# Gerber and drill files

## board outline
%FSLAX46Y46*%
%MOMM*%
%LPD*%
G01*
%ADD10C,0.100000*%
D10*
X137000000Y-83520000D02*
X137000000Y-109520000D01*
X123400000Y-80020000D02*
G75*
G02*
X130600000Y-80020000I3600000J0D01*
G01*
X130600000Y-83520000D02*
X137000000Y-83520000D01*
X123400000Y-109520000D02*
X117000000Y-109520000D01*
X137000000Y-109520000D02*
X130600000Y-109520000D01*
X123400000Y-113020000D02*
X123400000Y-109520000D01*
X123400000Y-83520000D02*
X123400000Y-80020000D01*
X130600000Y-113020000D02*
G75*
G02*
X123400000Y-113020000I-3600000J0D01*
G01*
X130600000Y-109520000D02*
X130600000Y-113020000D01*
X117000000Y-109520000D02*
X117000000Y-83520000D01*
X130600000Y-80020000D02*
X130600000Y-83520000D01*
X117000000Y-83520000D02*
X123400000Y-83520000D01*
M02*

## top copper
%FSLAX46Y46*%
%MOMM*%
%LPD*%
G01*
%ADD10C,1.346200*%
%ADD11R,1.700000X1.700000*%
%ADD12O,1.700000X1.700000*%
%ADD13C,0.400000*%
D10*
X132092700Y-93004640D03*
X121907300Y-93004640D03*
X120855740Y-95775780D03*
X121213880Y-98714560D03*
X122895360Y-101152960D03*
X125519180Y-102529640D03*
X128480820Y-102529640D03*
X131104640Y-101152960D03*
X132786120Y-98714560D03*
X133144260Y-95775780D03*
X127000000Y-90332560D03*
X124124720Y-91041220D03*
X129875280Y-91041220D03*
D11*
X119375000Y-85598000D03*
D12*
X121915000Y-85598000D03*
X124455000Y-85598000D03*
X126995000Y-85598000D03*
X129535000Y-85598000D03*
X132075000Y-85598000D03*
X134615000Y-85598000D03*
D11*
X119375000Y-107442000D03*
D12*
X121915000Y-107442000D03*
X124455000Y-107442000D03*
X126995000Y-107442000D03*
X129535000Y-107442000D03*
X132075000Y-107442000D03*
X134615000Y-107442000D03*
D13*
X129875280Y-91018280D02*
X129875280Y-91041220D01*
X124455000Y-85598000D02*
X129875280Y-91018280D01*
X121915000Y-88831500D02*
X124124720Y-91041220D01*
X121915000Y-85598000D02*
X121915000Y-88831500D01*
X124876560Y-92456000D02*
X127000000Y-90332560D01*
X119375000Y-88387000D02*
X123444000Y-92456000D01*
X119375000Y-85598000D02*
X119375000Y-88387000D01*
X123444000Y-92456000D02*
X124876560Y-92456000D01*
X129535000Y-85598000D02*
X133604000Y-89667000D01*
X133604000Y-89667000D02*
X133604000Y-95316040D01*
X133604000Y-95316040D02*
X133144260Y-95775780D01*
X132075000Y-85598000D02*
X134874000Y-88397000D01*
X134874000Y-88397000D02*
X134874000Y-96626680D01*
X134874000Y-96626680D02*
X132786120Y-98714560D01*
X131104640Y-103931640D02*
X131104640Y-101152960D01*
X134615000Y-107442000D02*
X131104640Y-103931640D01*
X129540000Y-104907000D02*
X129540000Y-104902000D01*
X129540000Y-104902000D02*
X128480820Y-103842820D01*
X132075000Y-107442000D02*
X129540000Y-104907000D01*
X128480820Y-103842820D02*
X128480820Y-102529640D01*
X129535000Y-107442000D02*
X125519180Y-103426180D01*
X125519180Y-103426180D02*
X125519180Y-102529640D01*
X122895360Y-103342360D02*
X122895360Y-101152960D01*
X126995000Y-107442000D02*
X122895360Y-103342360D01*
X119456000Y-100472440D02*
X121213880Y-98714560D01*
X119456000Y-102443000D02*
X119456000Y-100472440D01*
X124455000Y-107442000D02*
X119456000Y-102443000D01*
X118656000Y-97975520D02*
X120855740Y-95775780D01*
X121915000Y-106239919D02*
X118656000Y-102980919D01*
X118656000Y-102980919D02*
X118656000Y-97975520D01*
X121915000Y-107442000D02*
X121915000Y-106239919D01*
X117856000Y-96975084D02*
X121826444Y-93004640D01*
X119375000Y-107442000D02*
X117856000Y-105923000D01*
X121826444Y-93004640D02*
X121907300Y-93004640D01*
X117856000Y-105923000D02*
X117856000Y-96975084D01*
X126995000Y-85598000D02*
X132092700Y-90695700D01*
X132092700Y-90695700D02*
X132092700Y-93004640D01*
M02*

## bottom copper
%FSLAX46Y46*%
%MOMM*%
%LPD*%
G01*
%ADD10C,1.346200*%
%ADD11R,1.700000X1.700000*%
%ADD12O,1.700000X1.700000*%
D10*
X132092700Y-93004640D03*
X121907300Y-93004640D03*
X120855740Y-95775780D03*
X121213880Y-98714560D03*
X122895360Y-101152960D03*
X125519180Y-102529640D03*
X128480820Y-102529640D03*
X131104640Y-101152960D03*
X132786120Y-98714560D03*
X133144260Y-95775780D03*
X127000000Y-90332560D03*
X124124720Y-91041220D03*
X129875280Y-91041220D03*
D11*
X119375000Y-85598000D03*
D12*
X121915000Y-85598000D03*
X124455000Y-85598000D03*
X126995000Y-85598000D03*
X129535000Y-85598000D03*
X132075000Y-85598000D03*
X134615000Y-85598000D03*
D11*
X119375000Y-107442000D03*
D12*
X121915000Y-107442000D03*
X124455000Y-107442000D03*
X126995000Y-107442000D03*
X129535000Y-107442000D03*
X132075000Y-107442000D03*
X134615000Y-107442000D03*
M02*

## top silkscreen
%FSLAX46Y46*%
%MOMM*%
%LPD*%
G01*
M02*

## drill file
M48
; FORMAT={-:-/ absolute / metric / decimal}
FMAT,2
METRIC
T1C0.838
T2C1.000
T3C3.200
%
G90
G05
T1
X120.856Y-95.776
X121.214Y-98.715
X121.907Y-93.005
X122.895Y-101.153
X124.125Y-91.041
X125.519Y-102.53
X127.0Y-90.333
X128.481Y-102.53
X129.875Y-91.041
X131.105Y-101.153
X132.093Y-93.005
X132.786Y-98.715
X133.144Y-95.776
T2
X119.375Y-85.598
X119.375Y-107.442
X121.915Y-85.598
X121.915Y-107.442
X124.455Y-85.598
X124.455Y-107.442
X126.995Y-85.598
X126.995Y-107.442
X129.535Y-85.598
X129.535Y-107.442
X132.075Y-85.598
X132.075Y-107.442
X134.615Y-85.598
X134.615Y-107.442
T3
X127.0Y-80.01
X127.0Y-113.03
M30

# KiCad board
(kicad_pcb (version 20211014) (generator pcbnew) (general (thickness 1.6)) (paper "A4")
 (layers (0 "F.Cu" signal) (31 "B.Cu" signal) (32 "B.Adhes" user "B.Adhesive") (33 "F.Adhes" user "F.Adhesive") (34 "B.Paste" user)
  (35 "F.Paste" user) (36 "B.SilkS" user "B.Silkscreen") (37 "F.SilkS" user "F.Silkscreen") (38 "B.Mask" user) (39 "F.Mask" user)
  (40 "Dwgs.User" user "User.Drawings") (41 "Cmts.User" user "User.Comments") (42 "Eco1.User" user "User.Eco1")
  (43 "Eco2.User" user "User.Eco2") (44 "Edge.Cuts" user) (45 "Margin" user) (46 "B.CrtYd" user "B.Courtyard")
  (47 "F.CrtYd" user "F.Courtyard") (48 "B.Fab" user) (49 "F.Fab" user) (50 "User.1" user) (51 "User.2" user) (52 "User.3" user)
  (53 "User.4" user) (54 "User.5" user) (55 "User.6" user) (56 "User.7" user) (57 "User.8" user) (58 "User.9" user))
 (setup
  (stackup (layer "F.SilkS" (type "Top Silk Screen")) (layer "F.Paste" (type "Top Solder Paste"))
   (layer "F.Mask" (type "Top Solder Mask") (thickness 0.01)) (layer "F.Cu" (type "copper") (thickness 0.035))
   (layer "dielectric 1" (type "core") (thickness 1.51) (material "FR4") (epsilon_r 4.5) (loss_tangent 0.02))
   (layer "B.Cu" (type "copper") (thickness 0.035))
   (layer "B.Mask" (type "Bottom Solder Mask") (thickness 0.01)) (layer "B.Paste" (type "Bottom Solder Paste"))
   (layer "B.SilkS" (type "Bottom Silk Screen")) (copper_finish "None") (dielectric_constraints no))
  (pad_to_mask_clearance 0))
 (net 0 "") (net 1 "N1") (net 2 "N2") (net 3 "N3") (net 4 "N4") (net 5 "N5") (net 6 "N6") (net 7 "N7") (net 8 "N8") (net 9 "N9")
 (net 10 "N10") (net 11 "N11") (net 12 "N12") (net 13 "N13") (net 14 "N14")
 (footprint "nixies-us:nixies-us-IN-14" (layer "F.Cu") (at 127 96.52 180)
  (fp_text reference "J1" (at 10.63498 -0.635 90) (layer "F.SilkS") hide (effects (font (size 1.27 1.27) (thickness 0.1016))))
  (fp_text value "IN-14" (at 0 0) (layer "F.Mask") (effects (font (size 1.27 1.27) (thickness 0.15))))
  (pad "0" thru_hole circle (at -5.0927 3.51536 180) (size 1.3462 1.3462) (drill 0.8382) (layers *.Cu *.Mask) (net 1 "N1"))
  (pad "1" thru_hole circle (at 5.0927 3.51536 180) (size 1.3462 1.3462) (drill 0.8382) (layers *.Cu *.Mask) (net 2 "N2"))
  (pad "2" thru_hole circle (at 6.14426 0.74422 180) (size 1.3462 1.3462) (drill 0.8382) (layers *.Cu *.Mask) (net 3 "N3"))
  (pad "3" thru_hole circle (at 5.78612 -2.19456 180) (size 1.3462 1.3462) (drill 0.8382) (layers *.Cu *.Mask) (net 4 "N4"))
  (pad "4" thru_hole circle (at 4.10464 -4.63296 180) (size 1.3462 1.3462) (drill 0.8382) (layers *.Cu *.Mask) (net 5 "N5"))
  (pad "5" thru_hole circle (at 1.48082 -6.00964 180) (size 1.3462 1.3462) (drill 0.8382) (layers *.Cu *.Mask) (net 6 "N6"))
  (pad "6" thru_hole circle (at -1.48082 -6.00964 180) (size 1.3462 1.3462) (drill 0.8382) (layers *.Cu *.Mask) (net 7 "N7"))
  (pad "7" thru_hole circle (at -4.10464 -4.63296 180) (size 1.3462 1.3462) (drill 0.8382) (layers *.Cu *.Mask) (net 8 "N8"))
  (pad "8" thru_hole circle (at -5.78612 -2.19456 180) (size 1.3462 1.3462) (drill 0.8382) (layers *.Cu *.Mask) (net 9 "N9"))
  (pad "9" thru_hole circle (at -6.14426 0.74422 180) (size 1.3462 1.3462) (drill 0.8382) (layers *.Cu *.Mask) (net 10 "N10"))
  (pad "A" thru_hole circle (at 0 6.18744 180) (size 1.3462 1.3462) (drill 0.8382) (layers *.Cu *.Mask) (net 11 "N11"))
  (pad "LHDP" thru_hole circle (at 2.87528 5.47878 180) (size 1.3462 1.3462) (drill 0.8382) (layers *.Cu *.Mask) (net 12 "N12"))
  (pad "RHDP" thru_hole circle (at -2.87528 5.47878 180) (size 1.3462 1.3462) (drill 0.8382) (layers *.Cu *.Mask) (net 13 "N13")))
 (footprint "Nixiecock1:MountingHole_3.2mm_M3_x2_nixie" (layer "F.Cu") (at 127 96.52 90)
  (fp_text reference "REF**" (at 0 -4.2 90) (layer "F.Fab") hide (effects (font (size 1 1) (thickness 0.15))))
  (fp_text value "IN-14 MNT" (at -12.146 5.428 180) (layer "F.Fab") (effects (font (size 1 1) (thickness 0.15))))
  (pad "" np_thru_hole circle locked (at -16.51 0 90) (size 3.2 3.2) (drill 3.2) (layers F&B.Cu *.Mask))
  (pad "" np_thru_hole circle locked (at 16.51 0 90) (size 3.2 3.2) (drill 3.2) (layers F&B.Cu *.Mask)))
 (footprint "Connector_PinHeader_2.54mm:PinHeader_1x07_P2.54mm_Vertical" (layer "F.Cu") (at 119.375 85.598 90)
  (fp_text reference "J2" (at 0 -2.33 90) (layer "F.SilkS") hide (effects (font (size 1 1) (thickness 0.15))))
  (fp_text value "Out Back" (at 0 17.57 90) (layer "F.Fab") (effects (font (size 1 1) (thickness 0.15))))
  (pad "1" thru_hole rect (at 0 0 90) (size 1.7 1.7) (drill 1) (layers *.Cu *.Mask) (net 11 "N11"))
  (pad "2" thru_hole oval (at 0 2.54 90) (size 1.7 1.7) (drill 1) (layers *.Cu *.Mask) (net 12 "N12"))
  (pad "3" thru_hole oval (at 0 5.08 90) (size 1.7 1.7) (drill 1) (layers *.Cu *.Mask) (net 13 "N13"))
  (pad "4" thru_hole oval (at 0 7.62 90) (size 1.7 1.7) (drill 1) (layers *.Cu *.Mask) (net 1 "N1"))
  (pad "5" thru_hole oval (at 0 10.16 90) (size 1.7 1.7) (drill 1) (layers *.Cu *.Mask) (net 10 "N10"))
  (pad "6" thru_hole oval (at 0 12.7 90) (size 1.7 1.7) (drill 1) (layers *.Cu *.Mask) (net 9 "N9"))
  (pad "7" thru_hole oval (at 0 15.24 90) (size 1.7 1.7) (drill 1) (layers *.Cu *.Mask) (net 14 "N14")))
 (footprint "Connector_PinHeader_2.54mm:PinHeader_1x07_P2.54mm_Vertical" (layer "F.Cu") (at 119.375 107.442 90)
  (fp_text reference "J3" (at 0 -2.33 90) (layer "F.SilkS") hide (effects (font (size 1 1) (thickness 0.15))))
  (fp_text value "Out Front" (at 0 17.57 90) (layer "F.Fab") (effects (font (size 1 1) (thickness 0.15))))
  (pad "1" thru_hole rect (at 0 0 90) (size 1.7 1.7) (drill 1) (layers *.Cu *.Mask) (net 2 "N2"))
  (pad "2" thru_hole oval (at 0 2.54 90) (size 1.7 1.7) (drill 1) (layers *.Cu *.Mask) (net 3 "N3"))
  (pad "3" thru_hole oval (at 0 5.08 90) (size 1.7 1.7) (drill 1) (layers *.Cu *.Mask) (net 4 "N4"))
  (pad "4" thru_hole oval (at 0 7.62 90) (size 1.7 1.7) (drill 1) (layers *.Cu *.Mask) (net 5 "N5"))
  (pad "5" thru_hole oval (at 0 10.16 90) (size 1.7 1.7) (drill 1) (layers *.Cu *.Mask) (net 6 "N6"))
  (pad "6" thru_hole oval (at 0 12.7 90) (size 1.7 1.7) (drill 1) (layers *.Cu *.Mask) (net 7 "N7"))
  (pad "7" thru_hole oval (at 0 15.24 90) (size 1.7 1.7) (drill 1) (layers *.Cu *.Mask) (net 8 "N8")))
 (gr_line (start 137 83.52) (end 137 109.52) (layer "Edge.Cuts") (width 0.1))
 (gr_arc (start 123.4 80.02) (mid 127 76.42) (end 130.6 80.02) (layer "Edge.Cuts") (width 0.1))
 (gr_line (start 130.6 83.52) (end 137 83.52) (layer "Edge.Cuts") (width 0.1))
 (gr_line (start 123.4 109.52) (end 117 109.52) (layer "Edge.Cuts") (width 0.1))
 (gr_line (start 137 109.52) (end 130.6 109.52) (layer "Edge.Cuts") (width 0.1))
 (gr_line (start 123.4 113.02) (end 123.4 109.52) (layer "Edge.Cuts") (width 0.1))
 (gr_line (start 123.4 83.52) (end 123.4 80.02) (layer "Edge.Cuts") (width 0.1))
 (gr_arc (start 130.6 113.02) (mid 127 116.62) (end 123.4 113.02) (layer "Edge.Cuts") (width 0.1))
 (gr_line (start 130.6 109.52) (end 130.6 113.02) (layer "Edge.Cuts") (width 0.1))
 (gr_line (start 117 109.52) (end 117 83.52) (layer "Edge.Cuts") (width 0.1))
 (gr_line (start 130.6 80.02) (end 130.6 83.52) (layer "Edge.Cuts") (width 0.1))
 (gr_line (start 117 83.52) (end 123.4 83.52) (layer "Edge.Cuts") (width 0.1))
 (segment (start 129.87528 91.01828) (end 129.87528 91.04122) (width 0.4) (layer "F.Cu") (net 13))
 (segment (start 124.455 85.598) (end 129.87528 91.01828) (width 0.4) (layer "F.Cu") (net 13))
 (segment (start 121.915 88.8315) (end 124.12472 91.04122) (width 0.4) (layer "F.Cu") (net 12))
 (segment (start 121.915 85.598) (end 121.915 88.8315) (width 0.4) (layer "F.Cu") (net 12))
 (segment (start 124.87656 92.456) (end 127 90.33256) (width 0.4) (layer "F.Cu") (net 11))
 (segment (start 119.375 88.387) (end 123.444 92.456) (width 0.4) (layer "F.Cu") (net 11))
 (segment (start 119.375 85.598) (end 119.375 88.387) (width 0.4) (layer "F.Cu") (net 11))
 (segment (start 123.444 92.456) (end 124.87656 92.456) (width 0.4) (layer "F.Cu") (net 11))
 (segment (start 129.535 85.598) (end 133.604 89.667) (width 0.4) (layer "F.Cu") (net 10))
 (segment (start 133.604 89.667) (end 133.604 95.31604) (width 0.4) (layer "F.Cu") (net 10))
 (segment (start 133.604 95.31604) (end 133.14426 95.77578) (width 0.4) (layer "F.Cu") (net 10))
 (segment (start 132.075 85.598) (end 134.874 88.397) (width 0.4) (layer "F.Cu") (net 9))
 (segment (start 134.874 88.397) (end 134.874 96.62668) (width 0.4) (layer "F.Cu") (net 9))
 (segment (start 134.874 96.62668) (end 132.78612 98.71456) (width 0.4) (layer "F.Cu") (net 9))
 (segment (start 131.10464 103.93164) (end 131.10464 101.15296) (width 0.4) (layer "F.Cu") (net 8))
 (segment (start 134.615 107.442) (end 131.10464 103.93164) (width 0.4) (layer "F.Cu") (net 8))
 (segment (start 129.54 104.907) (end 129.54 104.902) (width 0.4) (layer "F.Cu") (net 7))
 (segment (start 129.54 104.902) (end 128.48082 103.84282) (width 0.4) (layer "F.Cu") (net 7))
 (segment (start 132.075 107.442) (end 129.54 104.907) (width 0.4) (layer "F.Cu") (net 7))
 (segment (start 128.48082 103.84282) (end 128.48082 102.52964) (width 0.4) (layer "F.Cu") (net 7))
 (segment (start 129.535 107.442) (end 125.51918 103.42618) (width 0.4) (layer "F.Cu") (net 6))
 (segment (start 125.51918 103.42618) (end 125.51918 102.52964) (width 0.4) (layer "F.Cu") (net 6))
 (segment (start 122.89536 103.34236) (end 122.89536 101.15296) (width 0.4) (layer "F.Cu") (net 5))
 (segment (start 126.995 107.442) (end 122.89536 103.34236) (width 0.4) (layer "F.Cu") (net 5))
 (segment (start 119.456 100.47244) (end 121.21388 98.71456) (width 0.4) (layer "F.Cu") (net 4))
 (segment (start 119.456 102.443) (end 119.456 100.47244) (width 0.4) (layer "F.Cu") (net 4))
 (segment (start 124.455 107.442) (end 119.456 102.443) (width 0.4) (layer "F.Cu") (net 4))
 (segment (start 118.656 97.97552) (end 120.85574 95.77578) (width 0.4) (layer "F.Cu") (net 3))
 (segment (start 121.915 106.239919) (end 118.656 102.980919) (width 0.4) (layer "F.Cu") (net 3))
 (segment (start 118.656 102.980919) (end 118.656 97.97552) (width 0.4) (layer "F.Cu") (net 3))
 (segment (start 121.915 107.442) (end 121.915 106.239919) (width 0.4) (layer "F.Cu") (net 3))
 (segment (start 117.856 96.975084) (end 121.826444 93.00464) (width 0.4) (layer "F.Cu") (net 2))
 (segment (start 119.375 107.442) (end 117.856 105.923) (width 0.4) (layer "F.Cu") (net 2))
 (segment (start 121.826444 93.00464) (end 121.9073 93.00464) (width 0.4) (layer "F.Cu") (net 2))
 (segment (start 117.856 105.923) (end 117.856 96.975084) (width 0.4) (layer "F.Cu") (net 2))
 (segment (start 126.995 85.598) (end 132.0927 90.6957) (width 0.4) (layer "F.Cu") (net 1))
 (segment (start 132.0927 90.6957) (end 132.0927 93.00464) (width 0.4) (layer "F.Cu") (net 1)))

